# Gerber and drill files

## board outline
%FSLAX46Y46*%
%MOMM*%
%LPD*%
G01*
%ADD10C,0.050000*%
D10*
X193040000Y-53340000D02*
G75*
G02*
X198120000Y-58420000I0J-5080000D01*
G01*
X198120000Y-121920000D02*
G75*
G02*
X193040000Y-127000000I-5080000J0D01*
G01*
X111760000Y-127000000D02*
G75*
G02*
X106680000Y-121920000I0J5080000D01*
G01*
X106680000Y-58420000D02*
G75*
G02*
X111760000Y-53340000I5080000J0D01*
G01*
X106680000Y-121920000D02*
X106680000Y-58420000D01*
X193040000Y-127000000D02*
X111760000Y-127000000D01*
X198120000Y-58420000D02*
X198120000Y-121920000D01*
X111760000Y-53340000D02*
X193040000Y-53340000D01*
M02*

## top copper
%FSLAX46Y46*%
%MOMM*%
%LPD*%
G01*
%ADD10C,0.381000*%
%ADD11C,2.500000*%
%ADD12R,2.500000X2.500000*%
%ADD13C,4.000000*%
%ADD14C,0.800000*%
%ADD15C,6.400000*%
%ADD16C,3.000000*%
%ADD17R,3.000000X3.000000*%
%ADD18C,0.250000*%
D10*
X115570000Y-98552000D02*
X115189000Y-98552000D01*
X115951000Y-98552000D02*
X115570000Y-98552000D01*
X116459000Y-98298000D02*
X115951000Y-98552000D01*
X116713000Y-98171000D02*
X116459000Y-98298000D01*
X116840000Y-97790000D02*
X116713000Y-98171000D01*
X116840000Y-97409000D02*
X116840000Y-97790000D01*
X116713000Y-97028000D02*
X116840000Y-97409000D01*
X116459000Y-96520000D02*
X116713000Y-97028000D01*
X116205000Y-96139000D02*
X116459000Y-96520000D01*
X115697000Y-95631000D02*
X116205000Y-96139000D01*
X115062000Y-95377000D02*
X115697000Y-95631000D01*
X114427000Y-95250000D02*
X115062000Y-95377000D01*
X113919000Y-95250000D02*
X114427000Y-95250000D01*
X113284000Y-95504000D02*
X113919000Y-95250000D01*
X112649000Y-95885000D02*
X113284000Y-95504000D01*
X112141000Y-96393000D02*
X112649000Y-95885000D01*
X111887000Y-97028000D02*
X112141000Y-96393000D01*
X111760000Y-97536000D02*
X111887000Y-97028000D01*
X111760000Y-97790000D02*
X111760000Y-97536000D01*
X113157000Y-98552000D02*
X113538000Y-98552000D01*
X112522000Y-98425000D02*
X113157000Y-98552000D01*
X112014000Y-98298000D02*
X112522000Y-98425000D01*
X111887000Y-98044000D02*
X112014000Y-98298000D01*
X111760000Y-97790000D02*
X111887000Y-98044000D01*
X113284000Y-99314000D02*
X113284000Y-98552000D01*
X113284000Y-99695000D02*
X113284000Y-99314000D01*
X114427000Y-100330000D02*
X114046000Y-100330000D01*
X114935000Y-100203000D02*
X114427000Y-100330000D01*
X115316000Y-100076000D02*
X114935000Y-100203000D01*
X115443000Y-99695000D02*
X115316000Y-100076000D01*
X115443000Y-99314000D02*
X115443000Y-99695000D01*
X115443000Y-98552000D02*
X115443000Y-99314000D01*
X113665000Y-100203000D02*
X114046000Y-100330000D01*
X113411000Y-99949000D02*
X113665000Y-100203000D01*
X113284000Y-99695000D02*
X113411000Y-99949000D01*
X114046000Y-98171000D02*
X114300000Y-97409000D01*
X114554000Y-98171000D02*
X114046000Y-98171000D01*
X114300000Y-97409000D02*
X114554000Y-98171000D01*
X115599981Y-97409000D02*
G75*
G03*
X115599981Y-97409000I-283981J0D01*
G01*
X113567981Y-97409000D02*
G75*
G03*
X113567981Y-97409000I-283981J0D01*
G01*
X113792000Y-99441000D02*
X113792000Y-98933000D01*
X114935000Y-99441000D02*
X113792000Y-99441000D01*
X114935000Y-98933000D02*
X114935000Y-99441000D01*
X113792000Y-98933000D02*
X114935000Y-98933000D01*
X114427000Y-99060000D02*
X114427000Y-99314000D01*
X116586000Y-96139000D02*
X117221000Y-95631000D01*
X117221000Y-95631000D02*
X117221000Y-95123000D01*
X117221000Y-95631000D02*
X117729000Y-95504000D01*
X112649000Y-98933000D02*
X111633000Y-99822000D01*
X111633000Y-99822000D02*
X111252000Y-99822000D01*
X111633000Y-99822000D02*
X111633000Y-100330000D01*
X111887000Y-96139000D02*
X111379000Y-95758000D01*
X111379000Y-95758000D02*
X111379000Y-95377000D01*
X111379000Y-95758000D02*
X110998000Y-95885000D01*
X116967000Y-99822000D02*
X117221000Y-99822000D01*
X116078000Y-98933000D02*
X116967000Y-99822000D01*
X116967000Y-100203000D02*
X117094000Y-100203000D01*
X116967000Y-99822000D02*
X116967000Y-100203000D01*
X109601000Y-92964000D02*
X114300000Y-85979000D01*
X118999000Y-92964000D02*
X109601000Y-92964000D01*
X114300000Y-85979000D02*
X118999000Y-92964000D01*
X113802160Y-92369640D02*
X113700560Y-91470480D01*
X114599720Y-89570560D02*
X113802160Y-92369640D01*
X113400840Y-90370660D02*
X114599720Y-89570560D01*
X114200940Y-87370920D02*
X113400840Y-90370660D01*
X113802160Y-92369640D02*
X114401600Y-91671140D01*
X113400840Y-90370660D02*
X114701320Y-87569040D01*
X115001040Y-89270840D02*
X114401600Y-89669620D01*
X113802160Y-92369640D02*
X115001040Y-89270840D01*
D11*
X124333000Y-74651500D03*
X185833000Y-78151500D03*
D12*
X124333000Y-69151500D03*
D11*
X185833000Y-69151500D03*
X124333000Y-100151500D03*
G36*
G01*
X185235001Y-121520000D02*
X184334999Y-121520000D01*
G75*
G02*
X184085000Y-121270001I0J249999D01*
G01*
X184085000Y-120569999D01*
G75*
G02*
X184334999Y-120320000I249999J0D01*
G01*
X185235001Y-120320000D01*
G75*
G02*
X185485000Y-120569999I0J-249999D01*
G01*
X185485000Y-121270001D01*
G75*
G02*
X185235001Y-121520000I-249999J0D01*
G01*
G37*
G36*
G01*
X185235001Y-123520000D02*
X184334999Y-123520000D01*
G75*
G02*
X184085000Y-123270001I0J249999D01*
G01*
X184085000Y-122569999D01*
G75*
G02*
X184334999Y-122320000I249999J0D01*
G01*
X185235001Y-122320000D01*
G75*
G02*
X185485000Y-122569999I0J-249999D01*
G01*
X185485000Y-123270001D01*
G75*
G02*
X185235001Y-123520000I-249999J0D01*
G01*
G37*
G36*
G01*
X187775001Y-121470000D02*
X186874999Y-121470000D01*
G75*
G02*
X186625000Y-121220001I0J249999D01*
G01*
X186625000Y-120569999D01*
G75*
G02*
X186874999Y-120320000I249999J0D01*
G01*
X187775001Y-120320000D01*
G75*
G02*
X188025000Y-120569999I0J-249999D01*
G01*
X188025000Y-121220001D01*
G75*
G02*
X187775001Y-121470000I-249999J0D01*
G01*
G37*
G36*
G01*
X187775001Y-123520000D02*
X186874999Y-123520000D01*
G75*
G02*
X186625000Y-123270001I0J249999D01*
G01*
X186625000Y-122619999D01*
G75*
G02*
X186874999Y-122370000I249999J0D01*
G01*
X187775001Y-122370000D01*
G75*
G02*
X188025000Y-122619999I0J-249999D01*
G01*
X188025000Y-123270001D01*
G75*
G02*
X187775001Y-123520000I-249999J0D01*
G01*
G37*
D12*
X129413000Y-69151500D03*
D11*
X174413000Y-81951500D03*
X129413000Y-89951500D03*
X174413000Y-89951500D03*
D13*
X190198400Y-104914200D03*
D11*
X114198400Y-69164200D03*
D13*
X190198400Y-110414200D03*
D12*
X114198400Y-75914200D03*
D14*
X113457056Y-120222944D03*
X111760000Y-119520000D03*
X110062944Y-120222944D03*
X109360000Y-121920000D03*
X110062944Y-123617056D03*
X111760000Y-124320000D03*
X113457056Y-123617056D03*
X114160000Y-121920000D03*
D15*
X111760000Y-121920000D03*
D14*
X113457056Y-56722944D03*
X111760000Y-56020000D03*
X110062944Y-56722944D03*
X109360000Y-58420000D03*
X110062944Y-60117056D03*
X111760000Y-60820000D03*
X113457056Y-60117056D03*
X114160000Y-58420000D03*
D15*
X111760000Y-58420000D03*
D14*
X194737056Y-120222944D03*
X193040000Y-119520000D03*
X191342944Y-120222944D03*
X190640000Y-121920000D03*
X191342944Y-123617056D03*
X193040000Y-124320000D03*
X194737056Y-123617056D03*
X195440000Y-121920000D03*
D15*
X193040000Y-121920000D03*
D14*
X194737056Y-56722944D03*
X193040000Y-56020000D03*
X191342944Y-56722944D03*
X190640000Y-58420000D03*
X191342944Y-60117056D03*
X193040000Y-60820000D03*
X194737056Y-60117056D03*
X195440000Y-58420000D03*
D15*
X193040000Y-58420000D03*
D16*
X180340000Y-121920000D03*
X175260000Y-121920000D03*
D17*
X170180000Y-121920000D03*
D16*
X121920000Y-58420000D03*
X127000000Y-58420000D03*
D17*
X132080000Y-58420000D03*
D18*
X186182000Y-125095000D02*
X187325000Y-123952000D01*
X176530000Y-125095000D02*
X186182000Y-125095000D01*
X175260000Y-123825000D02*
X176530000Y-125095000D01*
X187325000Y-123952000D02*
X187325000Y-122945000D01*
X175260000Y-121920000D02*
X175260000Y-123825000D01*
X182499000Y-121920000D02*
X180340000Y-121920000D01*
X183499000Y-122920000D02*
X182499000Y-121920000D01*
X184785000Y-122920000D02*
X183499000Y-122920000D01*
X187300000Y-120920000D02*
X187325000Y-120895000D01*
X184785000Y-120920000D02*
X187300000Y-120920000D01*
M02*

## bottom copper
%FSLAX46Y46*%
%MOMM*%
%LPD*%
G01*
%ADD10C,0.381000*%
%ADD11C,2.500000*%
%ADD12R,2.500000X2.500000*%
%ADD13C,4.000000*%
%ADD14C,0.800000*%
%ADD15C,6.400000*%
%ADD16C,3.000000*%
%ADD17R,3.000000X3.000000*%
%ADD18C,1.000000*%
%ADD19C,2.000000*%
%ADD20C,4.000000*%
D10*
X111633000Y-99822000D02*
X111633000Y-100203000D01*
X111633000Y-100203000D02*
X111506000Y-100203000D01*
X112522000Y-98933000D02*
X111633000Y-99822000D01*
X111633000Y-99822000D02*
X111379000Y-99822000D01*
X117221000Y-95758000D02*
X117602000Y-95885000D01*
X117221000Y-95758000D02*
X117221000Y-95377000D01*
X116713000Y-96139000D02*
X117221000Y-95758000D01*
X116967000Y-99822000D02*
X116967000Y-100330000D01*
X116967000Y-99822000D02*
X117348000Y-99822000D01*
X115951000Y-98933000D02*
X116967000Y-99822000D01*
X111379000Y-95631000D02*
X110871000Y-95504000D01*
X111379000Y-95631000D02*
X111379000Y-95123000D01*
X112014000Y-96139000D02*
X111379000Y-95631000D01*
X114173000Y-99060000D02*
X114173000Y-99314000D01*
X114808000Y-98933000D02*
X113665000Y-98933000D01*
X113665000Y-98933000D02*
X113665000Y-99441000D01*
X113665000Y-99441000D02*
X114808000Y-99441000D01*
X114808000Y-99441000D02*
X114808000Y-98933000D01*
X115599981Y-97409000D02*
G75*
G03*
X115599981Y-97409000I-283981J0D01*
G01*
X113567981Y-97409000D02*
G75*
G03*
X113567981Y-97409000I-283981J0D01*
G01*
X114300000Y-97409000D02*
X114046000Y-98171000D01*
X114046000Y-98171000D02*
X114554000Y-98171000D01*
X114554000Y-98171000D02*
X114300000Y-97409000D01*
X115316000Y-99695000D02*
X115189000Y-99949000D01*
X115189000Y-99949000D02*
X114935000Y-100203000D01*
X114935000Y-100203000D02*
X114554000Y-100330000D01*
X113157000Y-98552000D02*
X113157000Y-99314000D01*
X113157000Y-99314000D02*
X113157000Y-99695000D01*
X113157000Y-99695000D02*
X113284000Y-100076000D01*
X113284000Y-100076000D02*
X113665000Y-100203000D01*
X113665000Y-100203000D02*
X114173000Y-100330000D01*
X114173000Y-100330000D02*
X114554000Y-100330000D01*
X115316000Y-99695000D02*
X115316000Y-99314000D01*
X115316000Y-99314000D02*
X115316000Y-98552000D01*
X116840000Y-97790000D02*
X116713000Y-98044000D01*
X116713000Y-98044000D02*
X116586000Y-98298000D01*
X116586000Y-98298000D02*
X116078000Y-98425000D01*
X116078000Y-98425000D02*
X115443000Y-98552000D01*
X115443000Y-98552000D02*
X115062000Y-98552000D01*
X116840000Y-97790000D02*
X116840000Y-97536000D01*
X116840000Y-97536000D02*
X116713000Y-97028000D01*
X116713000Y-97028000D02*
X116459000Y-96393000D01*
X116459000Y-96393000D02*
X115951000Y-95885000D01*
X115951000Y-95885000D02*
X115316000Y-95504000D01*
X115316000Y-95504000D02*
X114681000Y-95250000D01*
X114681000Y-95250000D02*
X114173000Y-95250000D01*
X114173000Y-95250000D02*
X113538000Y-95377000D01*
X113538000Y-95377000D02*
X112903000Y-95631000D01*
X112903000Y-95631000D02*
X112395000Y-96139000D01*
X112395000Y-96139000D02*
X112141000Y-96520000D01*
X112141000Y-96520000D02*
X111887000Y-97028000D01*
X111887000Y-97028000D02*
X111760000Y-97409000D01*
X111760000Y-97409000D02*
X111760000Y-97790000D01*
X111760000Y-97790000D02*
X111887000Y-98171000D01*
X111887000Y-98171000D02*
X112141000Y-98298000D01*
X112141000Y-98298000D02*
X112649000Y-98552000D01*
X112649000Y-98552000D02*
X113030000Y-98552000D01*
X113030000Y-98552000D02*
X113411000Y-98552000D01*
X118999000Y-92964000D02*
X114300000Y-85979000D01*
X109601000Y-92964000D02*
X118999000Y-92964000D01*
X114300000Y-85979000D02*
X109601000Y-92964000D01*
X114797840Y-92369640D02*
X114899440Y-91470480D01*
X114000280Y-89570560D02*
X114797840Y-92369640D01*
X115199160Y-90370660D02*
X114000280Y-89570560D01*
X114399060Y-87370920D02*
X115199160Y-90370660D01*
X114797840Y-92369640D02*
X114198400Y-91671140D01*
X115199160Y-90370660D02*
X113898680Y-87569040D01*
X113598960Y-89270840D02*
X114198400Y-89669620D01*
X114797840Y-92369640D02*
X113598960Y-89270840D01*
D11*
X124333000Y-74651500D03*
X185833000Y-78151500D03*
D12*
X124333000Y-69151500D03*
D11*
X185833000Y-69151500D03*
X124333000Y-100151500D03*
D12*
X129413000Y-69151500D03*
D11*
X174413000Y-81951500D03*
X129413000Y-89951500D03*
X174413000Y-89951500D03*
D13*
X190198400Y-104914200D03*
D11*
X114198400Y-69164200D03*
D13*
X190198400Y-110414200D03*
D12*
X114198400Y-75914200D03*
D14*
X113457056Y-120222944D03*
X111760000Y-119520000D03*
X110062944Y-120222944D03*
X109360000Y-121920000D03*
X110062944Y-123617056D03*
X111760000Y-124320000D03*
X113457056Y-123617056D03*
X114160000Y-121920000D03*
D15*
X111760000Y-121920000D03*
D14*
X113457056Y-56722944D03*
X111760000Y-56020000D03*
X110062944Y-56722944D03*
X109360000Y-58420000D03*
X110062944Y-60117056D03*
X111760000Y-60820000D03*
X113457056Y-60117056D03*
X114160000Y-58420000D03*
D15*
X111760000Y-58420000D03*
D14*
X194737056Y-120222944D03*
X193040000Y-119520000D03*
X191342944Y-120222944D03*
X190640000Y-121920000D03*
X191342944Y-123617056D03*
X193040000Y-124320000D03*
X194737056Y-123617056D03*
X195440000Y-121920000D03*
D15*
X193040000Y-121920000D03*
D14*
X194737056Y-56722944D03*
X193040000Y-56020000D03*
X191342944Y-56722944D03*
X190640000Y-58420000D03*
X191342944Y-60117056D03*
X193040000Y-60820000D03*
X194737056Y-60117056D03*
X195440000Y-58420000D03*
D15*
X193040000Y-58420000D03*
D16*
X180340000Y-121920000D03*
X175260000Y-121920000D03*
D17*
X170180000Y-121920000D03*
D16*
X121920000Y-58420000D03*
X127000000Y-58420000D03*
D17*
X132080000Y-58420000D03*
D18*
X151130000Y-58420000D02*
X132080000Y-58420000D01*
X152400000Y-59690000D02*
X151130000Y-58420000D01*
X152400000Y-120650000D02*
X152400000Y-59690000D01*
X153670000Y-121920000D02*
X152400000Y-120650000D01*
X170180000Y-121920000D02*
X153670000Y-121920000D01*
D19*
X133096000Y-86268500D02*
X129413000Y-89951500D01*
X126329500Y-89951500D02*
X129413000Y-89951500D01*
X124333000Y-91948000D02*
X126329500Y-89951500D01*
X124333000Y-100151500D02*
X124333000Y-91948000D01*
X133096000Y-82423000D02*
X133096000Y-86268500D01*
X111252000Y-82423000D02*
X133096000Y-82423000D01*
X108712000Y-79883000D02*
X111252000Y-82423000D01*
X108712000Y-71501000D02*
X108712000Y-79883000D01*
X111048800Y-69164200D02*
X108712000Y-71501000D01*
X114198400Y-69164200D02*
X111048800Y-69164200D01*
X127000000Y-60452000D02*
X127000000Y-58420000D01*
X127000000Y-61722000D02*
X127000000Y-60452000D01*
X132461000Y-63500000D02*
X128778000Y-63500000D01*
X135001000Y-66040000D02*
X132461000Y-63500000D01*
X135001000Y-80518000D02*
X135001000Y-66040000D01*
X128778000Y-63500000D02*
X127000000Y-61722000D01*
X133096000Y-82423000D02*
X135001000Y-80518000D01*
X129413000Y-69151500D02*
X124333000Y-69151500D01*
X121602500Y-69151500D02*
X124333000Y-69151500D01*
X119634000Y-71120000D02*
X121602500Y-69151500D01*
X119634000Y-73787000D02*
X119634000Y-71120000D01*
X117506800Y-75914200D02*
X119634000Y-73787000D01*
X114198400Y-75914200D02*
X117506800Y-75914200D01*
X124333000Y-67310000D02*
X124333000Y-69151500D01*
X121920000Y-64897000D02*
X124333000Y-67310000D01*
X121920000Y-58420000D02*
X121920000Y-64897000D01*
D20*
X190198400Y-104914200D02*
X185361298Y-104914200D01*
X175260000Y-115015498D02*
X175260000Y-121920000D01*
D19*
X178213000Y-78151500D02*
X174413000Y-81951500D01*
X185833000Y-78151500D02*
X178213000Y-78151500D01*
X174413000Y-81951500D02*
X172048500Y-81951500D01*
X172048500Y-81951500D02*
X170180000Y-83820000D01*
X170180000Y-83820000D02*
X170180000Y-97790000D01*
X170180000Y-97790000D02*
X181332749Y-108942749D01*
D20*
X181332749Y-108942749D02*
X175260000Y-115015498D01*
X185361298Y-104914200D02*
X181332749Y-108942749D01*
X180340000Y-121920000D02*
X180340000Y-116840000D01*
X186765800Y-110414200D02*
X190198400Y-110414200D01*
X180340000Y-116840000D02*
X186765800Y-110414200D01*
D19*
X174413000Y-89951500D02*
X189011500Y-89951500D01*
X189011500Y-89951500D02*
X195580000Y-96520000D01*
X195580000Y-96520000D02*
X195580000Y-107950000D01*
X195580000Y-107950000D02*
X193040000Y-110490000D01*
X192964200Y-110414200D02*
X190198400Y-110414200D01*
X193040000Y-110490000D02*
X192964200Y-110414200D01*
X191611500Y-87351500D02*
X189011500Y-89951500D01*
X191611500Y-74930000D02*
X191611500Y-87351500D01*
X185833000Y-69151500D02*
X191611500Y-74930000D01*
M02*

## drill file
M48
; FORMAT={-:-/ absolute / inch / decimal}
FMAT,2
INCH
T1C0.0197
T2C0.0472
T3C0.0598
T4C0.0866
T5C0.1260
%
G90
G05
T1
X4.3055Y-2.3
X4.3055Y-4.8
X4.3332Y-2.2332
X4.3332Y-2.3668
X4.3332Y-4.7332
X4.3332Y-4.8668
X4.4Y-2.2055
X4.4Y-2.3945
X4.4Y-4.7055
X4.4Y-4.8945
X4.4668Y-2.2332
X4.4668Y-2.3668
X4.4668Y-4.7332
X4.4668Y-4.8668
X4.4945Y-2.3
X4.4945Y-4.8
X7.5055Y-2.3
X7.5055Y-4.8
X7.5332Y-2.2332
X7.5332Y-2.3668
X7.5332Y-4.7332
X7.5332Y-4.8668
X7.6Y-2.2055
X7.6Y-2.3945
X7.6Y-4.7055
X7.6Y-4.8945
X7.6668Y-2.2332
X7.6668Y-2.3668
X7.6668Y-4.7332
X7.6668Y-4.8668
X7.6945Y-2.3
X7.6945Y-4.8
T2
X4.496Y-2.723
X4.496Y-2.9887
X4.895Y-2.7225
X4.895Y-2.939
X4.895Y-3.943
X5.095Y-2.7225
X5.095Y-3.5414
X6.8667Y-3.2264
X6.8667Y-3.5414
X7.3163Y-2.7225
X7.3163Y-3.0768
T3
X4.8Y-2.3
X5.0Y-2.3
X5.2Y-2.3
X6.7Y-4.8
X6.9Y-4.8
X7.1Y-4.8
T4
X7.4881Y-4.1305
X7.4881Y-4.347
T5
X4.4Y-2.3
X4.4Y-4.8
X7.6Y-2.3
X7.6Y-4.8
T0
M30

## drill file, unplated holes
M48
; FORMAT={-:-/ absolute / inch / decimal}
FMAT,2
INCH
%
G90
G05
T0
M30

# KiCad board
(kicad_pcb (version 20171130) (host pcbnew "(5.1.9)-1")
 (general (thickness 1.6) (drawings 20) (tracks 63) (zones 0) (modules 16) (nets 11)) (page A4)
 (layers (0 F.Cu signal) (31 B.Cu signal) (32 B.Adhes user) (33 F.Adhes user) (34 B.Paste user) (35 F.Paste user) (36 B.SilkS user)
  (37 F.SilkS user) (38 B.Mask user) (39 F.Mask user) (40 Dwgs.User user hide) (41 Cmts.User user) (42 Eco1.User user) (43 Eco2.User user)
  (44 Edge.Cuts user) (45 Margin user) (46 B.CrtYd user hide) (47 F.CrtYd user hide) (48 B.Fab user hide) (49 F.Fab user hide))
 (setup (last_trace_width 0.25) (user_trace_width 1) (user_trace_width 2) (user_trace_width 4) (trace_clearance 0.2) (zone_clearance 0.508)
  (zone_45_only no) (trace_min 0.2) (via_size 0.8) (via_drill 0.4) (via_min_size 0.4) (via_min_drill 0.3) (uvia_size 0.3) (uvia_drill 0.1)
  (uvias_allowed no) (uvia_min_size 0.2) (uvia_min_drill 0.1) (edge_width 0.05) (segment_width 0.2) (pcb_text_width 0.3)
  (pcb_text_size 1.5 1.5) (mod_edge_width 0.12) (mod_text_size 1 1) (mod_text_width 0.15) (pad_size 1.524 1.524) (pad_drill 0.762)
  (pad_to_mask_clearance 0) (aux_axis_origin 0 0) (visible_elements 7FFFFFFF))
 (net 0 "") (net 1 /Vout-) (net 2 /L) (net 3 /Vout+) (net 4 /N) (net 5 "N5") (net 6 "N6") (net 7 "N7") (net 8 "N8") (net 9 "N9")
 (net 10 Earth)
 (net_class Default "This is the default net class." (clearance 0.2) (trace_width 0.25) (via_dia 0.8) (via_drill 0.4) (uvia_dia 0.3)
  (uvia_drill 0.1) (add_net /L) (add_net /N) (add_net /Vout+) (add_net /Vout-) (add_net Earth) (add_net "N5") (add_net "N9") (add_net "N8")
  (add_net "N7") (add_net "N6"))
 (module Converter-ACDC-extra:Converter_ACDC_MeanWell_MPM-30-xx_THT (layer F.Cu) (at 155.083 84.1515)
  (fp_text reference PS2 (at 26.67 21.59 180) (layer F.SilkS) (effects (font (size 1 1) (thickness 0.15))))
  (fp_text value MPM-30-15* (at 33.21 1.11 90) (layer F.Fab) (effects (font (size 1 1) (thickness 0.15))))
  (pad ~ thru_hole circle (at -30.75 -9.5) (size 2.5 2.5) (drill 1.2) (layers *.Cu *.Mask))
  (pad 4 thru_hole circle (at 30.75 -6 90) (size 2.5 2.5) (drill 1.2) (layers *.Cu *.Mask) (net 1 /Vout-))
  (pad 1 thru_hole rect (at -30.75 -15) (size 2.5 2.5) (drill 1.2) (layers *.Cu *.Mask) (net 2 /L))
  (pad 3 thru_hole circle (at 30.75 -15) (size 2.5 2.5) (drill 1.2) (layers *.Cu *.Mask) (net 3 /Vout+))
  (pad 2 thru_hole circle (at -30.75 16) (size 2.5 2.5) (drill 1.2) (layers *.Cu *.Mask) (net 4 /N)))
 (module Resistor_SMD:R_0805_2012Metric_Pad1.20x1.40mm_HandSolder (layer F.Cu) (at 184.785 121.92 90)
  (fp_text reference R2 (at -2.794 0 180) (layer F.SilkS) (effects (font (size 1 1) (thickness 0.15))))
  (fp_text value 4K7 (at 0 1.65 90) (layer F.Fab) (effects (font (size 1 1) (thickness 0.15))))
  (pad 2 smd roundrect (at 1 0 90) (size 1.2 1.4) (layers F.Cu F.Paste F.Mask) (roundrect_rratio 0.2083325) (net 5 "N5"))
  (pad 1 smd roundrect (at -1 0 90) (size 1.2 1.4) (layers F.Cu F.Paste F.Mask) (roundrect_rratio 0.2083325) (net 3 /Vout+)))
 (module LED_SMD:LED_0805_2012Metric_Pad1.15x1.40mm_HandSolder (layer F.Cu) (at 187.325 121.92 90)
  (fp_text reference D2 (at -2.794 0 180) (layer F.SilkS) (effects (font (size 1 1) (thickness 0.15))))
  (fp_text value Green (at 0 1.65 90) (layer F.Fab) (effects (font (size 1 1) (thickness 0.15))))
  (pad 2 smd roundrect (at 1.025 0 90) (size 1.15 1.4) (layers F.Cu F.Paste F.Mask) (roundrect_rratio 0.2173904347826087) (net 5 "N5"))
  (pad 1 smd roundrect (at -1.025 0 90) (size 1.15 1.4) (layers F.Cu F.Paste F.Mask) (roundrect_rratio 0.2173904347826087) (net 1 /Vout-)))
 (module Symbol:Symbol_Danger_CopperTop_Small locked (layer B.Cu) (at 114.3 97.79 180)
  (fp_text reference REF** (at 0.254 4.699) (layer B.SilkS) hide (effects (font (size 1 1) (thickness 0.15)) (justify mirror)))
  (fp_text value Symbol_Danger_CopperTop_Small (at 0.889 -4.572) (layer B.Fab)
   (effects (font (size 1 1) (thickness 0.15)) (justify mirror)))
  (fp_line (start 2.667 -2.032) (end 2.667 -2.413) (layer B.Cu) (width 0.381))
  (fp_line (start 2.667 -2.413) (end 2.794 -2.413) (layer B.Cu) (width 0.381))
  (fp_line (start 1.778 -1.143) (end 2.667 -2.032) (layer B.Cu) (width 0.381))
  (fp_line (start 2.667 -2.032) (end 2.921 -2.032) (layer B.Cu) (width 0.381))
  (fp_line (start -2.921 2.032) (end -3.302 1.905) (layer B.Cu) (width 0.381))
  (fp_line (start -2.921 2.032) (end -2.921 2.413) (layer B.Cu) (width 0.381))
  (fp_line (start -2.413 1.651) (end -2.921 2.032) (layer B.Cu) (width 0.381))
  (fp_line (start -2.667 -2.032) (end -2.667 -2.54) (layer B.Cu) (width 0.381))
  (fp_line (start -2.667 -2.032) (end -3.048 -2.032) (layer B.Cu) (width 0.381))
  (fp_line (start -1.651 -1.143) (end -2.667 -2.032) (layer B.Cu) (width 0.381))
  (fp_line (start 2.921 2.159) (end 3.429 2.286) (layer B.Cu) (width 0.381))
  (fp_line (start 2.921 2.159) (end 2.921 2.667) (layer B.Cu) (width 0.381))
  (fp_line (start 2.286 1.651) (end 2.921 2.159) (layer B.Cu) (width 0.381))
  (fp_line (start 0.127 -1.27) (end 0.127 -1.524) (layer B.Cu) (width 0.381))
  (fp_line (start -0.508 -1.143) (end 0.635 -1.143) (layer B.Cu) (width 0.381))
  (fp_line (start 0.635 -1.143) (end 0.635 -1.651) (layer B.Cu) (width 0.381))
  (fp_line (start 0.635 -1.651) (end -0.508 -1.651) (layer B.Cu) (width 0.381))
  (fp_line (start -0.508 -1.651) (end -0.508 -1.143) (layer B.Cu) (width 0.381))
  (fp_circle (center -1.016 0.381) (end -1.27 0.254) (layer B.Cu) (width 0.381))
  (fp_circle (center 1.016 0.381) (end 1.27 0.254) (layer B.Cu) (width 0.381))
  (fp_line (start 0 0.381) (end 0.254 -0.381) (layer B.Cu) (width 0.381))
  (fp_line (start 0.254 -0.381) (end -0.254 -0.381) (layer B.Cu) (width 0.381))
  (fp_line (start -0.254 -0.381) (end 0 0.381) (layer B.Cu) (width 0.381))
  (fp_line (start -1.016 -1.905) (end -0.889 -2.159) (layer B.Cu) (width 0.381))
  (fp_line (start -0.889 -2.159) (end -0.635 -2.413) (layer B.Cu) (width 0.381))
  (fp_line (start -0.635 -2.413) (end -0.254 -2.54) (layer B.Cu) (width 0.381))
  (fp_line (start 1.143 -0.762) (end 1.143 -1.524) (layer B.Cu) (width 0.381))
  (fp_line (start 1.143 -1.524) (end 1.143 -1.905) (layer B.Cu) (width 0.381))
  (fp_line (start 1.143 -1.905) (end 1.016 -2.286) (layer B.Cu) (width 0.381))
  (fp_line (start 1.016 -2.286) (end 0.635 -2.413) (layer B.Cu) (width 0.381))
  (fp_line (start 0.635 -2.413) (end 0.127 -2.54) (layer B.Cu) (width 0.381))
  (fp_line (start 0.127 -2.54) (end -0.254 -2.54) (layer B.Cu) (width 0.381))
  (fp_line (start -1.016 -1.905) (end -1.016 -1.524) (layer B.Cu) (width 0.381))
  (fp_line (start -1.016 -1.524) (end -1.016 -0.762) (layer B.Cu) (width 0.381))
  (fp_line (start -2.54 0) (end -2.413 -0.254) (layer B.Cu) (width 0.381))
  (fp_line (start -2.413 -0.254) (end -2.286 -0.508) (layer B.Cu) (width 0.381))
  (fp_line (start -2.286 -0.508) (end -1.778 -0.635) (layer B.Cu) (width 0.381))
  (fp_line (start -1.778 -0.635) (end -1.143 -0.762) (layer B.Cu) (width 0.381))
  (fp_line (start -1.143 -0.762) (end -0.762 -0.762) (layer B.Cu) (width 0.381))
  (fp_line (start -2.54 0) (end -2.54 0.254) (layer B.Cu) (width 0.381))
  (fp_line (start -2.54 0.254) (end -2.413 0.762) (layer B.Cu) (width 0.381))
  (fp_line (start -2.413 0.762) (end -2.159 1.397) (layer B.Cu) (width 0.381))
  (fp_line (start -2.159 1.397) (end -1.651 1.905) (layer B.Cu) (width 0.381))
  (fp_line (start -1.651 1.905) (end -1.016 2.286) (layer B.Cu) (width 0.381))
  (fp_line (start -1.016 2.286) (end -0.381 2.54) (layer B.Cu) (width 0.381))
  (fp_line (start -0.381 2.54) (end 0.127 2.54) (layer B.Cu) (width 0.381))
  (fp_line (start 0.127 2.54) (end 0.762 2.413) (layer B.Cu) (width 0.381))
  (fp_line (start 0.762 2.413) (end 1.397 2.159) (layer B.Cu) (width 0.381))
  (fp_line (start 1.397 2.159) (end 1.905 1.651) (layer B.Cu) (width 0.381))
  (fp_line (start 1.905 1.651) (end 2.159 1.27) (layer B.Cu) (width 0.381))
  (fp_line (start 2.159 1.27) (end 2.413 0.762) (layer B.Cu) (width 0.381))
  (fp_line (start 2.413 0.762) (end 2.54 0.381) (layer B.Cu) (width 0.381))
  (fp_line (start 2.54 0.381) (end 2.54 0) (layer B.Cu) (width 0.381))
  (fp_line (start 2.54 0) (end 2.413 -0.381) (layer B.Cu) (width 0.381))
  (fp_line (start 2.413 -0.381) (end 2.159 -0.508) (layer B.Cu) (width 0.381))
  (fp_line (start 2.159 -0.508) (end 1.651 -0.762) (layer B.Cu) (width 0.381))
  (fp_line (start 1.651 -0.762) (end 1.27 -0.762) (layer B.Cu) (width 0.381))
  (fp_line (start 1.27 -0.762) (end 0.889 -0.762) (layer B.Cu) (width 0.381)))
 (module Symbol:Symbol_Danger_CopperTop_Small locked (layer F.Cu) (at 114.3 97.79)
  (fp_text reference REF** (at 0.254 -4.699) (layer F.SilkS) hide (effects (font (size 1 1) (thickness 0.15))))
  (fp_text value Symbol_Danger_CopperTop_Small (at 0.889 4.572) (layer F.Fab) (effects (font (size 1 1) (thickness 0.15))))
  (fp_line (start 1.27 0.762) (end 0.889 0.762) (layer F.Cu) (width 0.381))
  (fp_line (start 1.651 0.762) (end 1.27 0.762) (layer F.Cu) (width 0.381))
  (fp_line (start 2.159 0.508) (end 1.651 0.762) (layer F.Cu) (width 0.381))
  (fp_line (start 2.413 0.381) (end 2.159 0.508) (layer F.Cu) (width 0.381))
  (fp_line (start 2.54 0) (end 2.413 0.381) (layer F.Cu) (width 0.381))
  (fp_line (start 2.54 -0.381) (end 2.54 0) (layer F.Cu) (width 0.381))
  (fp_line (start 2.413 -0.762) (end 2.54 -0.381) (layer F.Cu) (width 0.381))
  (fp_line (start 2.159 -1.27) (end 2.413 -0.762) (layer F.Cu) (width 0.381))
  (fp_line (start 1.905 -1.651) (end 2.159 -1.27) (layer F.Cu) (width 0.381))
  (fp_line (start 1.397 -2.159) (end 1.905 -1.651) (layer F.Cu) (width 0.381))
  (fp_line (start 0.762 -2.413) (end 1.397 -2.159) (layer F.Cu) (width 0.381))
  (fp_line (start 0.127 -2.54) (end 0.762 -2.413) (layer F.Cu) (width 0.381))
  (fp_line (start -0.381 -2.54) (end 0.127 -2.54) (layer F.Cu) (width 0.381))
  (fp_line (start -1.016 -2.286) (end -0.381 -2.54) (layer F.Cu) (width 0.381))
  (fp_line (start -1.651 -1.905) (end -1.016 -2.286) (layer F.Cu) (width 0.381))
  (fp_line (start -2.159 -1.397) (end -1.651 -1.905) (layer F.Cu) (width 0.381))
  (fp_line (start -2.413 -0.762) (end -2.159 -1.397) (layer F.Cu) (width 0.381))
  (fp_line (start -2.54 -0.254) (end -2.413 -0.762) (layer F.Cu) (width 0.381))
  (fp_line (start -2.54 0) (end -2.54 -0.254) (layer F.Cu) (width 0.381))
  (fp_line (start -1.143 0.762) (end -0.762 0.762) (layer F.Cu) (width 0.381))
  (fp_line (start -1.778 0.635) (end -1.143 0.762) (layer F.Cu) (width 0.381))
  (fp_line (start -2.286 0.508) (end -1.778 0.635) (layer F.Cu) (width 0.381))
  (fp_line (start -2.413 0.254) (end -2.286 0.508) (layer F.Cu) (width 0.381))
  (fp_line (start -2.54 0) (end -2.413 0.254) (layer F.Cu) (width 0.381))
  (fp_line (start -1.016 1.524) (end -1.016 0.762) (layer F.Cu) (width 0.381))
  (fp_line (start -1.016 1.905) (end -1.016 1.524) (layer F.Cu) (width 0.381))
  (fp_line (start 0.127 2.54) (end -0.254 2.54) (layer F.Cu) (width 0.381))
  (fp_line (start 0.635 2.413) (end 0.127 2.54) (layer F.Cu) (width 0.381))
  (fp_line (start 1.016 2.286) (end 0.635 2.413) (layer F.Cu) (width 0.381))
  (fp_line (start 1.143 1.905) (end 1.016 2.286) (layer F.Cu) (width 0.381))
  (fp_line (start 1.143 1.524) (end 1.143 1.905) (layer F.Cu) (width 0.381))
  (fp_line (start 1.143 0.762) (end 1.143 1.524) (layer F.Cu) (width 0.381))
  (fp_line (start -0.635 2.413) (end -0.254 2.54) (layer F.Cu) (width 0.381))
  (fp_line (start -0.889 2.159) (end -0.635 2.413) (layer F.Cu) (width 0.381))
  (fp_line (start -1.016 1.905) (end -0.889 2.159) (layer F.Cu) (width 0.381))
  (fp_line (start -0.254 0.381) (end 0 -0.381) (layer F.Cu) (width 0.381))
  (fp_line (start 0.254 0.381) (end -0.254 0.381) (layer F.Cu) (width 0.381))
  (fp_line (start 0 -0.381) (end 0.254 0.381) (layer F.Cu) (width 0.381))
  (fp_circle (center 1.016 -0.381) (end 1.27 -0.254) (layer F.Cu) (width 0.381))
  (fp_circle (center -1.016 -0.381) (end -1.27 -0.254) (layer F.Cu) (width 0.381))
  (fp_line (start -0.508 1.651) (end -0.508 1.143) (layer F.Cu) (width 0.381))
  (fp_line (start 0.635 1.651) (end -0.508 1.651) (layer F.Cu) (width 0.381))
  (fp_line (start 0.635 1.143) (end 0.635 1.651) (layer F.Cu) (width 0.381))
  (fp_line (start -0.508 1.143) (end 0.635 1.143) (layer F.Cu) (width 0.381))
  (fp_line (start 0.127 1.27) (end 0.127 1.524) (layer F.Cu) (width 0.381))
  (fp_line (start 2.286 -1.651) (end 2.921 -2.159) (layer F.Cu) (width 0.381))
  (fp_line (start 2.921 -2.159) (end 2.921 -2.667) (layer F.Cu) (width 0.381))
  (fp_line (start 2.921 -2.159) (end 3.429 -2.286) (layer F.Cu) (width 0.381))
  (fp_line (start -1.651 1.143) (end -2.667 2.032) (layer F.Cu) (width 0.381))
  (fp_line (start -2.667 2.032) (end -3.048 2.032) (layer F.Cu) (width 0.381))
  (fp_line (start -2.667 2.032) (end -2.667 2.54) (layer F.Cu) (width 0.381))
  (fp_line (start -2.413 -1.651) (end -2.921 -2.032) (layer F.Cu) (width 0.381))
  (fp_line (start -2.921 -2.032) (end -2.921 -2.413) (layer F.Cu) (width 0.381))
  (fp_line (start -2.921 -2.032) (end -3.302 -1.905) (layer F.Cu) (width 0.381))
  (fp_line (start 2.667 2.032) (end 2.921 2.032) (layer F.Cu) (width 0.381))
  (fp_line (start 1.778 1.143) (end 2.667 2.032) (layer F.Cu) (width 0.381))
  (fp_line (start 2.667 2.413) (end 2.794 2.413) (layer F.Cu) (width 0.381))
  (fp_line (start 2.667 2.032) (end 2.667 2.413) (layer F.Cu) (width 0.381)))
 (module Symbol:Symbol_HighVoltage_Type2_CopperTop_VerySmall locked (layer B.Cu) (at 114.3 90.17 180)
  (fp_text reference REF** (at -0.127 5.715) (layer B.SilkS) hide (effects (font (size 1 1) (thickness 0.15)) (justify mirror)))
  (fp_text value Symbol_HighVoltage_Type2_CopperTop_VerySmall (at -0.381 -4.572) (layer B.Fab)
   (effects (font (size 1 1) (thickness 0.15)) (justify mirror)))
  (fp_line (start -4.699 -2.794) (end 0 4.191) (layer B.Cu) (width 0.381))
  (fp_line (start 4.699 -2.794) (end -4.699 -2.794) (layer B.Cu) (width 0.381))
  (fp_line (start 0 4.191) (end 4.699 -2.794) (layer B.Cu) (width 0.381))
  (fp_line (start -0.49784 -2.19964) (end -0.59944 -1.30048) (layer B.Cu) (width 0.381))
  (fp_line (start 0.29972 0.59944) (end -0.49784 -2.19964) (layer B.Cu) (width 0.381))
  (fp_line (start -0.89916 -0.20066) (end 0.29972 0.59944) (layer B.Cu) (width 0.381))
  (fp_line (start -0.09906 2.79908) (end -0.89916 -0.20066) (layer B.Cu) (width 0.381))
  (fp_line (start -0.49784 -2.19964) (end 0.1016 -1.50114) (layer B.Cu) (width 0.381))
  (fp_line (start -0.89916 -0.20066) (end 0.40132 2.60096) (layer B.Cu) (width 0.381))
  (fp_line (start 0.70104 0.89916) (end 0.1016 0.50038) (layer B.Cu) (width 0.381))
  (fp_line (start -0.49784 -2.19964) (end 0.70104 0.89916) (layer B.Cu) (width 0.381)))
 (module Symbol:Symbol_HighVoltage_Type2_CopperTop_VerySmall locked (layer F.Cu) (at 114.3 90.17)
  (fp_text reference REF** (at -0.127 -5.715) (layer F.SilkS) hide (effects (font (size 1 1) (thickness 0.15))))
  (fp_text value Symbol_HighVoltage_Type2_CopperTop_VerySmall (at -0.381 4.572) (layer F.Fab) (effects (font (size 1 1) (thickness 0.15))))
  (fp_line (start -4.699 2.794) (end 0 -4.191) (layer F.Cu) (width 0.381))
  (fp_line (start 4.699 2.794) (end -4.699 2.794) (layer F.Cu) (width 0.381))
  (fp_line (start 0 -4.191) (end 4.699 2.794) (layer F.Cu) (width 0.381))
  (fp_line (start -0.49784 2.19964) (end -0.59944 1.30048) (layer F.Cu) (width 0.381))
  (fp_line (start 0.29972 -0.59944) (end -0.49784 2.19964) (layer F.Cu) (width 0.381))
  (fp_line (start -0.89916 0.20066) (end 0.29972 -0.59944) (layer F.Cu) (width 0.381))
  (fp_line (start -0.09906 -2.79908) (end -0.89916 0.20066) (layer F.Cu) (width 0.381))
  (fp_line (start -0.49784 2.19964) (end 0.1016 1.50114) (layer F.Cu) (width 0.381))
  (fp_line (start -0.89916 0.20066) (end 0.40132 -2.60096) (layer F.Cu) (width 0.381))
  (fp_line (start 0.70104 -0.89916) (end 0.1016 -0.50038) (layer F.Cu) (width 0.381))
  (fp_line (start -0.49784 2.19964) (end 0.70104 -0.89916) (layer F.Cu) (width 0.381)))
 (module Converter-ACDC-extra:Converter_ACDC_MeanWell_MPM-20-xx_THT (layer F.Cu) (at 152.213 79.5515)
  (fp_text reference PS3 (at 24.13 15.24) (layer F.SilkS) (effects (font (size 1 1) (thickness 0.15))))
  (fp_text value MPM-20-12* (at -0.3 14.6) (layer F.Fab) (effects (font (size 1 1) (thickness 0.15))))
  (pad 1 thru_hole rect (at -22.8 -10.4) (size 2.5 2.5) (drill 1.2) (layers *.Cu *.Mask) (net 2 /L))
  (pad 4 thru_hole circle (at 22.2 2.4) (size 2.5 2.5) (drill 1.2) (layers *.Cu *.Mask) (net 1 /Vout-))
  (pad 2 thru_hole circle (at -22.8 10.4) (size 2.5 2.5) (drill 1.2) (layers *.Cu *.Mask) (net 4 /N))
  (pad 3 thru_hole circle (at 22.2 10.4) (size 2.5 2.5) (drill 1.2) (layers *.Cu *.Mask) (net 3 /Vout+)))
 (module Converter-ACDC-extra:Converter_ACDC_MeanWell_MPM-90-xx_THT (layer F.Cu) (at 152.4 90.17)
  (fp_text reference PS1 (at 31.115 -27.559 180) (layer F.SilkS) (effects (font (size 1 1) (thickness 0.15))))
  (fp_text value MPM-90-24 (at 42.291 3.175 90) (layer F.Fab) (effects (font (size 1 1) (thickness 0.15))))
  (pad 4 thru_hole circle (at 37.7984 14.7442) (size 4 4) (drill 2.2) (layers *.Cu *.Mask) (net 1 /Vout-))
  (pad 2 thru_hole circle (at -38.2016 -21.0058) (size 2.5 2.5) (drill 1.2) (layers *.Cu *.Mask) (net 4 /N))
  (pad 3 thru_hole circle (at 37.7984 20.2442) (size 4 4) (drill 2.2) (layers *.Cu *.Mask) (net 3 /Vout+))
  (pad 1 thru_hole rect (at -38.2016 -14.2558) (size 2.5 2.5) (drill 1.2) (layers *.Cu *.Mask) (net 2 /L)))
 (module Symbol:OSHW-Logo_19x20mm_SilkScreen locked (layer B.Cu) (at 152.4 109.22 180)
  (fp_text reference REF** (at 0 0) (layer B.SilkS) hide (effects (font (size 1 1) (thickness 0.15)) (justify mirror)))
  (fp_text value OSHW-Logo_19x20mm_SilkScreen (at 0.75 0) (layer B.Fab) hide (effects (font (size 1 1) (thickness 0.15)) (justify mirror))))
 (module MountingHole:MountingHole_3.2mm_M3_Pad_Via (layer F.Cu) (at 111.76 121.92)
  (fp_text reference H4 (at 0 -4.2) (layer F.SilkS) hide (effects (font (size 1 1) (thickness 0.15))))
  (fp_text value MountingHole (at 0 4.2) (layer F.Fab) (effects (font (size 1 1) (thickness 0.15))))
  (pad 1 thru_hole circle (at 1.697056 -1.697056) (size 0.8 0.8) (drill 0.5) (layers *.Cu *.Mask) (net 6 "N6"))
  (pad 1 thru_hole circle (at 0 -2.4) (size 0.8 0.8) (drill 0.5) (layers *.Cu *.Mask) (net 6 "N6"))
  (pad 1 thru_hole circle (at -1.697056 -1.697056) (size 0.8 0.8) (drill 0.5) (layers *.Cu *.Mask) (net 6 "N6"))
  (pad 1 thru_hole circle (at -2.4 0) (size 0.8 0.8) (drill 0.5) (layers *.Cu *.Mask) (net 6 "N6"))
  (pad 1 thru_hole circle (at -1.697056 1.697056) (size 0.8 0.8) (drill 0.5) (layers *.Cu *.Mask) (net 6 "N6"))
  (pad 1 thru_hole circle (at 0 2.4) (size 0.8 0.8) (drill 0.5) (layers *.Cu *.Mask) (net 6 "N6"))
  (pad 1 thru_hole circle (at 1.697056 1.697056) (size 0.8 0.8) (drill 0.5) (layers *.Cu *.Mask) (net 6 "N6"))
  (pad 1 thru_hole circle (at 2.4 0) (size 0.8 0.8) (drill 0.5) (layers *.Cu *.Mask) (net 6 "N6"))
  (pad 1 thru_hole circle (at 0 0) (size 6.4 6.4) (drill 3.2) (layers *.Cu *.Mask) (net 6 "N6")))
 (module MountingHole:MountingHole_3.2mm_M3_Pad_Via (layer F.Cu) (at 111.76 58.42)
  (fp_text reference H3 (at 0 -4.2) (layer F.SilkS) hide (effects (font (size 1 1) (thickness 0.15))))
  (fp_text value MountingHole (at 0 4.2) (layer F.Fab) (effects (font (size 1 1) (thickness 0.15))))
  (pad 1 thru_hole circle (at 1.697056 -1.697056) (size 0.8 0.8) (drill 0.5) (layers *.Cu *.Mask) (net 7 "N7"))
  (pad 1 thru_hole circle (at 0 -2.4) (size 0.8 0.8) (drill 0.5) (layers *.Cu *.Mask) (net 7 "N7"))
  (pad 1 thru_hole circle (at -1.697056 -1.697056) (size 0.8 0.8) (drill 0.5) (layers *.Cu *.Mask) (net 7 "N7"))
  (pad 1 thru_hole circle (at -2.4 0) (size 0.8 0.8) (drill 0.5) (layers *.Cu *.Mask) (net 7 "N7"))
  (pad 1 thru_hole circle (at -1.697056 1.697056) (size 0.8 0.8) (drill 0.5) (layers *.Cu *.Mask) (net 7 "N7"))
  (pad 1 thru_hole circle (at 0 2.4) (size 0.8 0.8) (drill 0.5) (layers *.Cu *.Mask) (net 7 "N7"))
  (pad 1 thru_hole circle (at 1.697056 1.697056) (size 0.8 0.8) (drill 0.5) (layers *.Cu *.Mask) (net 7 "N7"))
  (pad 1 thru_hole circle (at 2.4 0) (size 0.8 0.8) (drill 0.5) (layers *.Cu *.Mask) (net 7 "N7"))
  (pad 1 thru_hole circle (at 0 0) (size 6.4 6.4) (drill 3.2) (layers *.Cu *.Mask) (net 7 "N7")))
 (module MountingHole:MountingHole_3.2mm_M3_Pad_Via (layer F.Cu) (at 193.04 121.92)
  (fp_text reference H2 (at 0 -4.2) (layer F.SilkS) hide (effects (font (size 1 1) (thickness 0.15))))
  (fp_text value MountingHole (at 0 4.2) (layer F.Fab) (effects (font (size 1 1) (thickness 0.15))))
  (pad 1 thru_hole circle (at 1.697056 -1.697056) (size 0.8 0.8) (drill 0.5) (layers *.Cu *.Mask) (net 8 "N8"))
  (pad 1 thru_hole circle (at 0 -2.4) (size 0.8 0.8) (drill 0.5) (layers *.Cu *.Mask) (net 8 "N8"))
  (pad 1 thru_hole circle (at -1.697056 -1.697056) (size 0.8 0.8) (drill 0.5) (layers *.Cu *.Mask) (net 8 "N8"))
  (pad 1 thru_hole circle (at -2.4 0) (size 0.8 0.8) (drill 0.5) (layers *.Cu *.Mask) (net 8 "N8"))
  (pad 1 thru_hole circle (at -1.697056 1.697056) (size 0.8 0.8) (drill 0.5) (layers *.Cu *.Mask) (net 8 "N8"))
  (pad 1 thru_hole circle (at 0 2.4) (size 0.8 0.8) (drill 0.5) (layers *.Cu *.Mask) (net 8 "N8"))
  (pad 1 thru_hole circle (at 1.697056 1.697056) (size 0.8 0.8) (drill 0.5) (layers *.Cu *.Mask) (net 8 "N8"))
  (pad 1 thru_hole circle (at 2.4 0) (size 0.8 0.8) (drill 0.5) (layers *.Cu *.Mask) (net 8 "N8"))
  (pad 1 thru_hole circle (at 0 0) (size 6.4 6.4) (drill 3.2) (layers *.Cu *.Mask) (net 8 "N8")))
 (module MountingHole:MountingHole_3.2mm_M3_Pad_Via (layer F.Cu) (at 193.04 58.42)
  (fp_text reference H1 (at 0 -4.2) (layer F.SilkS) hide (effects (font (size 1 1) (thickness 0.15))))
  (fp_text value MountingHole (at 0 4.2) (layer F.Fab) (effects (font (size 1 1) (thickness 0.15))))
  (pad 1 thru_hole circle (at 1.697056 -1.697056) (size 0.8 0.8) (drill 0.5) (layers *.Cu *.Mask) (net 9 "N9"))
  (pad 1 thru_hole circle (at 0 -2.4) (size 0.8 0.8) (drill 0.5) (layers *.Cu *.Mask) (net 9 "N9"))
  (pad 1 thru_hole circle (at -1.697056 -1.697056) (size 0.8 0.8) (drill 0.5) (layers *.Cu *.Mask) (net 9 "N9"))
  (pad 1 thru_hole circle (at -2.4 0) (size 0.8 0.8) (drill 0.5) (layers *.Cu *.Mask) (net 9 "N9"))
  (pad 1 thru_hole circle (at -1.697056 1.697056) (size 0.8 0.8) (drill 0.5) (layers *.Cu *.Mask) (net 9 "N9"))
  (pad 1 thru_hole circle (at 0 2.4) (size 0.8 0.8) (drill 0.5) (layers *.Cu *.Mask) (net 9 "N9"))
  (pad 1 thru_hole circle (at 1.697056 1.697056) (size 0.8 0.8) (drill 0.5) (layers *.Cu *.Mask) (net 9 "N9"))
  (pad 1 thru_hole circle (at 2.4 0) (size 0.8 0.8) (drill 0.5) (layers *.Cu *.Mask) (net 9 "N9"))
  (pad 1 thru_hole circle (at 0 0) (size 6.4 6.4) (drill 3.2) (layers *.Cu *.Mask) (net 9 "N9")))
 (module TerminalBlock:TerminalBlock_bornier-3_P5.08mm (layer F.Cu) (at 170.18 121.92)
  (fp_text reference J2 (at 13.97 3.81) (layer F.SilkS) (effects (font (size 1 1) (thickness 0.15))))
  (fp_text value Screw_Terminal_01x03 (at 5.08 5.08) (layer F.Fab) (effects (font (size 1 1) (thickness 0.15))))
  (pad 3 thru_hole circle (at 10.16 0) (size 3 3) (drill 1.52) (layers *.Cu *.Mask) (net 3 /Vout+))
  (pad 2 thru_hole circle (at 5.08 0) (size 3 3) (drill 1.52) (layers *.Cu *.Mask) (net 1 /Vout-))
  (pad 1 thru_hole rect (at 0 0) (size 3 3) (drill 1.52) (layers *.Cu *.Mask) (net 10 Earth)))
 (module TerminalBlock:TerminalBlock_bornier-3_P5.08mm (layer F.Cu) (at 132.08 58.42 180)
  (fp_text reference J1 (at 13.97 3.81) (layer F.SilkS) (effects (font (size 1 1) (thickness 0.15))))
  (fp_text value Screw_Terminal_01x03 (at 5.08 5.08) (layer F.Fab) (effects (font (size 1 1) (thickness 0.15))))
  (pad 3 thru_hole circle (at 10.16 0 180) (size 3 3) (drill 1.52) (layers *.Cu *.Mask) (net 2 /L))
  (pad 2 thru_hole circle (at 5.08 0 180) (size 3 3) (drill 1.52) (layers *.Cu *.Mask) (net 4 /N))
  (pad 1 thru_hole rect (at 0 0 180) (size 3 3) (drill 1.52) (layers *.Cu *.Mask) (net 10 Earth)))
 (gr_arc (start 193.04 58.42) (end 198.12 58.42) (angle -90) (layer Edge.Cuts) (width 0.05))
 (gr_arc (start 193.04 121.92) (end 193.04 127) (angle -90) (layer Edge.Cuts) (width 0.05))
 (gr_arc (start 111.76 121.92) (end 106.68 121.92) (angle -90) (layer Edge.Cuts) (width 0.05))
 (gr_arc (start 111.76 58.42) (end 111.76 53.34) (angle -90) (layer Edge.Cuts) (width 0.05))
 (gr_line (start 106.68 121.92) (end 106.68 58.42) (layer Edge.Cuts) (width 0.05))
 (gr_line (start 193.04 127) (end 111.76 127) (layer Edge.Cuts) (width 0.05))
 (gr_line (start 198.12 58.42) (end 198.12 121.92) (layer Edge.Cuts) (width 0.05))
 (gr_line (start 111.76 53.34) (end 193.04 53.34) (layer Edge.Cuts) (width 0.05))
 (segment (start 151.13 58.42) (end 132.08 58.42) (width 1) (layer B.Cu) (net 10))
 (segment (start 152.4 59.69) (end 151.13 58.42) (width 1) (layer B.Cu) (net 10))
 (segment (start 152.4 120.65) (end 152.4 59.69) (width 1) (layer B.Cu) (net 10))
 (segment (start 153.67 121.92) (end 152.4 120.65) (width 1) (layer B.Cu) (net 10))
 (segment (start 170.18 121.92) (end 153.67 121.92) (width 1) (layer B.Cu) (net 10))
 (segment (start 133.096 86.2685) (end 129.413 89.9515) (width 2) (layer B.Cu) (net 4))
 (segment (start 126.3295 89.9515) (end 129.413 89.9515) (width 2) (layer B.Cu) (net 4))
 (segment (start 124.333 91.948) (end 126.3295 89.9515) (width 2) (layer B.Cu) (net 4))
 (segment (start 124.333 100.1515) (end 124.333 91.948) (width 2) (layer B.Cu) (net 4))
 (segment (start 133.096 82.423) (end 133.096 86.2685) (width 2) (layer B.Cu) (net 4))
 (segment (start 111.252 82.423) (end 133.096 82.423) (width 2) (layer B.Cu) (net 4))
 (segment (start 108.712 79.883) (end 111.252 82.423) (width 2) (layer B.Cu) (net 4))
 (segment (start 108.712 71.501) (end 108.712 79.883) (width 2) (layer B.Cu) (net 4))
 (segment (start 111.0488 69.1642) (end 108.712 71.501) (width 2) (layer B.Cu) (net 4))
 (segment (start 114.1984 69.1642) (end 111.0488 69.1642) (width 2) (layer B.Cu) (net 4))
 (segment (start 127 60.452) (end 127 58.42) (width 2) (layer B.Cu) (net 4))
 (segment (start 127 61.722) (end 127 60.452) (width 2) (layer B.Cu) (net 4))
 (segment (start 132.461 63.5) (end 128.778 63.5) (width 2) (layer B.Cu) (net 4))
 (segment (start 135.001 66.04) (end 132.461 63.5) (width 2) (layer B.Cu) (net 4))
 (segment (start 135.001 80.518) (end 135.001 66.04) (width 2) (layer B.Cu) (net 4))
 (segment (start 128.778 63.5) (end 127 61.722) (width 2) (layer B.Cu) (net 4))
 (segment (start 133.096 82.423) (end 135.001 80.518) (width 2) (layer B.Cu) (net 4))
 (segment (start 129.413 69.1515) (end 124.333 69.1515) (width 2) (layer B.Cu) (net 2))
 (segment (start 121.6025 69.1515) (end 124.333 69.1515) (width 2) (layer B.Cu) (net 2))
 (segment (start 119.634 71.12) (end 121.6025 69.1515) (width 2) (layer B.Cu) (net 2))
 (segment (start 119.634 73.787) (end 119.634 71.12) (width 2) (layer B.Cu) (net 2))
 (segment (start 117.5068 75.9142) (end 119.634 73.787) (width 2) (layer B.Cu) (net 2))
 (segment (start 114.1984 75.9142) (end 117.5068 75.9142) (width 2) (layer B.Cu) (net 2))
 (segment (start 124.333 67.31) (end 124.333 69.1515) (width 2) (layer B.Cu) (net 2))
 (segment (start 121.92 64.897) (end 124.333 67.31) (width 2) (layer B.Cu) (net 2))
 (segment (start 121.92 58.42) (end 121.92 64.897) (width 2) (layer B.Cu) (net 2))
 (segment (start 190.1984 104.9142) (end 185.361298 104.9142) (width 4) (layer B.Cu) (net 1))
 (segment (start 175.26 115.015498) (end 175.26 121.92) (width 4) (layer B.Cu) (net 1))
 (segment (start 178.213 78.1515) (end 174.413 81.9515) (width 2) (layer B.Cu) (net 1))
 (segment (start 185.833 78.1515) (end 178.213 78.1515) (width 2) (layer B.Cu) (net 1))
 (segment (start 174.413 81.9515) (end 172.0485 81.9515) (width 2) (layer B.Cu) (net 1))
 (segment (start 172.0485 81.9515) (end 170.18 83.82) (width 2) (layer B.Cu) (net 1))
 (segment (start 170.18 83.82) (end 170.18 97.79) (width 2) (layer B.Cu) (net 1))
 (segment (start 170.18 97.79) (end 181.332749 108.942749) (width 2) (layer B.Cu) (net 1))
 (segment (start 181.332749 108.942749) (end 175.26 115.015498) (width 4) (layer B.Cu) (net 1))
 (segment (start 185.361298 104.9142) (end 181.332749 108.942749) (width 4) (layer B.Cu) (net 1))
 (segment (start 186.182 125.095) (end 187.325 123.952) (width 0.25) (layer F.Cu) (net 1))
 (segment (start 176.53 125.095) (end 186.182 125.095) (width 0.25) (layer F.Cu) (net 1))
 (segment (start 175.26 123.825) (end 176.53 125.095) (width 0.25) (layer F.Cu) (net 1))
 (segment (start 187.325 123.952) (end 187.325 122.945) (width 0.25) (layer F.Cu) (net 1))
 (segment (start 175.26 121.92) (end 175.26 123.825) (width 0.25) (layer F.Cu) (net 1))
 (segment (start 180.34 121.92) (end 180.34 116.84) (width 4) (layer B.Cu) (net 3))
 (segment (start 186.7658 110.4142) (end 190.1984 110.4142) (width 4) (layer B.Cu) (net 3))
 (segment (start 180.34 116.84) (end 186.7658 110.4142) (width 4) (layer B.Cu) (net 3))
 (segment (start 174.413 89.9515) (end 189.0115 89.9515) (width 2) (layer B.Cu) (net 3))
 (segment (start 189.0115 89.9515) (end 195.58 96.52) (width 2) (layer B.Cu) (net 3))
 (segment (start 195.58 96.52) (end 195.58 107.95) (width 2) (layer B.Cu) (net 3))
 (segment (start 195.58 107.95) (end 193.04 110.49) (width 2) (layer B.Cu) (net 3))
 (segment (start 192.9642 110.4142) (end 190.1984 110.4142) (width 2) (layer B.Cu) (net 3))
 (segment (start 193.04 110.49) (end 192.9642 110.4142) (width 2) (layer B.Cu) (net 3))
 (segment (start 191.6115 87.3515) (end 189.0115 89.9515) (width 2) (layer B.Cu) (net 3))
 (segment (start 191.6115 74.93) (end 191.6115 87.3515) (width 2) (layer B.Cu) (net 3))
 (segment (start 182.499 121.92) (end 180.34 121.92) (width 0.25) (layer F.Cu) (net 3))
 (segment (start 183.499 122.92) (end 182.499 121.92) (width 0.25) (layer F.Cu) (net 3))
 (segment (start 184.785 122.92) (end 183.499 122.92) (width 0.25) (layer F.Cu) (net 3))
 (segment (start 185.833 69.1515) (end 191.6115 74.93) (width 2) (layer B.Cu) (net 3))
 (segment (start 187.3 120.92) (end 187.325 120.895) (width 0.25) (layer F.Cu) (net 5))
 (segment (start 184.785 120.92) (end 187.3 120.92) (width 0.25) (layer F.Cu) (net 5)))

